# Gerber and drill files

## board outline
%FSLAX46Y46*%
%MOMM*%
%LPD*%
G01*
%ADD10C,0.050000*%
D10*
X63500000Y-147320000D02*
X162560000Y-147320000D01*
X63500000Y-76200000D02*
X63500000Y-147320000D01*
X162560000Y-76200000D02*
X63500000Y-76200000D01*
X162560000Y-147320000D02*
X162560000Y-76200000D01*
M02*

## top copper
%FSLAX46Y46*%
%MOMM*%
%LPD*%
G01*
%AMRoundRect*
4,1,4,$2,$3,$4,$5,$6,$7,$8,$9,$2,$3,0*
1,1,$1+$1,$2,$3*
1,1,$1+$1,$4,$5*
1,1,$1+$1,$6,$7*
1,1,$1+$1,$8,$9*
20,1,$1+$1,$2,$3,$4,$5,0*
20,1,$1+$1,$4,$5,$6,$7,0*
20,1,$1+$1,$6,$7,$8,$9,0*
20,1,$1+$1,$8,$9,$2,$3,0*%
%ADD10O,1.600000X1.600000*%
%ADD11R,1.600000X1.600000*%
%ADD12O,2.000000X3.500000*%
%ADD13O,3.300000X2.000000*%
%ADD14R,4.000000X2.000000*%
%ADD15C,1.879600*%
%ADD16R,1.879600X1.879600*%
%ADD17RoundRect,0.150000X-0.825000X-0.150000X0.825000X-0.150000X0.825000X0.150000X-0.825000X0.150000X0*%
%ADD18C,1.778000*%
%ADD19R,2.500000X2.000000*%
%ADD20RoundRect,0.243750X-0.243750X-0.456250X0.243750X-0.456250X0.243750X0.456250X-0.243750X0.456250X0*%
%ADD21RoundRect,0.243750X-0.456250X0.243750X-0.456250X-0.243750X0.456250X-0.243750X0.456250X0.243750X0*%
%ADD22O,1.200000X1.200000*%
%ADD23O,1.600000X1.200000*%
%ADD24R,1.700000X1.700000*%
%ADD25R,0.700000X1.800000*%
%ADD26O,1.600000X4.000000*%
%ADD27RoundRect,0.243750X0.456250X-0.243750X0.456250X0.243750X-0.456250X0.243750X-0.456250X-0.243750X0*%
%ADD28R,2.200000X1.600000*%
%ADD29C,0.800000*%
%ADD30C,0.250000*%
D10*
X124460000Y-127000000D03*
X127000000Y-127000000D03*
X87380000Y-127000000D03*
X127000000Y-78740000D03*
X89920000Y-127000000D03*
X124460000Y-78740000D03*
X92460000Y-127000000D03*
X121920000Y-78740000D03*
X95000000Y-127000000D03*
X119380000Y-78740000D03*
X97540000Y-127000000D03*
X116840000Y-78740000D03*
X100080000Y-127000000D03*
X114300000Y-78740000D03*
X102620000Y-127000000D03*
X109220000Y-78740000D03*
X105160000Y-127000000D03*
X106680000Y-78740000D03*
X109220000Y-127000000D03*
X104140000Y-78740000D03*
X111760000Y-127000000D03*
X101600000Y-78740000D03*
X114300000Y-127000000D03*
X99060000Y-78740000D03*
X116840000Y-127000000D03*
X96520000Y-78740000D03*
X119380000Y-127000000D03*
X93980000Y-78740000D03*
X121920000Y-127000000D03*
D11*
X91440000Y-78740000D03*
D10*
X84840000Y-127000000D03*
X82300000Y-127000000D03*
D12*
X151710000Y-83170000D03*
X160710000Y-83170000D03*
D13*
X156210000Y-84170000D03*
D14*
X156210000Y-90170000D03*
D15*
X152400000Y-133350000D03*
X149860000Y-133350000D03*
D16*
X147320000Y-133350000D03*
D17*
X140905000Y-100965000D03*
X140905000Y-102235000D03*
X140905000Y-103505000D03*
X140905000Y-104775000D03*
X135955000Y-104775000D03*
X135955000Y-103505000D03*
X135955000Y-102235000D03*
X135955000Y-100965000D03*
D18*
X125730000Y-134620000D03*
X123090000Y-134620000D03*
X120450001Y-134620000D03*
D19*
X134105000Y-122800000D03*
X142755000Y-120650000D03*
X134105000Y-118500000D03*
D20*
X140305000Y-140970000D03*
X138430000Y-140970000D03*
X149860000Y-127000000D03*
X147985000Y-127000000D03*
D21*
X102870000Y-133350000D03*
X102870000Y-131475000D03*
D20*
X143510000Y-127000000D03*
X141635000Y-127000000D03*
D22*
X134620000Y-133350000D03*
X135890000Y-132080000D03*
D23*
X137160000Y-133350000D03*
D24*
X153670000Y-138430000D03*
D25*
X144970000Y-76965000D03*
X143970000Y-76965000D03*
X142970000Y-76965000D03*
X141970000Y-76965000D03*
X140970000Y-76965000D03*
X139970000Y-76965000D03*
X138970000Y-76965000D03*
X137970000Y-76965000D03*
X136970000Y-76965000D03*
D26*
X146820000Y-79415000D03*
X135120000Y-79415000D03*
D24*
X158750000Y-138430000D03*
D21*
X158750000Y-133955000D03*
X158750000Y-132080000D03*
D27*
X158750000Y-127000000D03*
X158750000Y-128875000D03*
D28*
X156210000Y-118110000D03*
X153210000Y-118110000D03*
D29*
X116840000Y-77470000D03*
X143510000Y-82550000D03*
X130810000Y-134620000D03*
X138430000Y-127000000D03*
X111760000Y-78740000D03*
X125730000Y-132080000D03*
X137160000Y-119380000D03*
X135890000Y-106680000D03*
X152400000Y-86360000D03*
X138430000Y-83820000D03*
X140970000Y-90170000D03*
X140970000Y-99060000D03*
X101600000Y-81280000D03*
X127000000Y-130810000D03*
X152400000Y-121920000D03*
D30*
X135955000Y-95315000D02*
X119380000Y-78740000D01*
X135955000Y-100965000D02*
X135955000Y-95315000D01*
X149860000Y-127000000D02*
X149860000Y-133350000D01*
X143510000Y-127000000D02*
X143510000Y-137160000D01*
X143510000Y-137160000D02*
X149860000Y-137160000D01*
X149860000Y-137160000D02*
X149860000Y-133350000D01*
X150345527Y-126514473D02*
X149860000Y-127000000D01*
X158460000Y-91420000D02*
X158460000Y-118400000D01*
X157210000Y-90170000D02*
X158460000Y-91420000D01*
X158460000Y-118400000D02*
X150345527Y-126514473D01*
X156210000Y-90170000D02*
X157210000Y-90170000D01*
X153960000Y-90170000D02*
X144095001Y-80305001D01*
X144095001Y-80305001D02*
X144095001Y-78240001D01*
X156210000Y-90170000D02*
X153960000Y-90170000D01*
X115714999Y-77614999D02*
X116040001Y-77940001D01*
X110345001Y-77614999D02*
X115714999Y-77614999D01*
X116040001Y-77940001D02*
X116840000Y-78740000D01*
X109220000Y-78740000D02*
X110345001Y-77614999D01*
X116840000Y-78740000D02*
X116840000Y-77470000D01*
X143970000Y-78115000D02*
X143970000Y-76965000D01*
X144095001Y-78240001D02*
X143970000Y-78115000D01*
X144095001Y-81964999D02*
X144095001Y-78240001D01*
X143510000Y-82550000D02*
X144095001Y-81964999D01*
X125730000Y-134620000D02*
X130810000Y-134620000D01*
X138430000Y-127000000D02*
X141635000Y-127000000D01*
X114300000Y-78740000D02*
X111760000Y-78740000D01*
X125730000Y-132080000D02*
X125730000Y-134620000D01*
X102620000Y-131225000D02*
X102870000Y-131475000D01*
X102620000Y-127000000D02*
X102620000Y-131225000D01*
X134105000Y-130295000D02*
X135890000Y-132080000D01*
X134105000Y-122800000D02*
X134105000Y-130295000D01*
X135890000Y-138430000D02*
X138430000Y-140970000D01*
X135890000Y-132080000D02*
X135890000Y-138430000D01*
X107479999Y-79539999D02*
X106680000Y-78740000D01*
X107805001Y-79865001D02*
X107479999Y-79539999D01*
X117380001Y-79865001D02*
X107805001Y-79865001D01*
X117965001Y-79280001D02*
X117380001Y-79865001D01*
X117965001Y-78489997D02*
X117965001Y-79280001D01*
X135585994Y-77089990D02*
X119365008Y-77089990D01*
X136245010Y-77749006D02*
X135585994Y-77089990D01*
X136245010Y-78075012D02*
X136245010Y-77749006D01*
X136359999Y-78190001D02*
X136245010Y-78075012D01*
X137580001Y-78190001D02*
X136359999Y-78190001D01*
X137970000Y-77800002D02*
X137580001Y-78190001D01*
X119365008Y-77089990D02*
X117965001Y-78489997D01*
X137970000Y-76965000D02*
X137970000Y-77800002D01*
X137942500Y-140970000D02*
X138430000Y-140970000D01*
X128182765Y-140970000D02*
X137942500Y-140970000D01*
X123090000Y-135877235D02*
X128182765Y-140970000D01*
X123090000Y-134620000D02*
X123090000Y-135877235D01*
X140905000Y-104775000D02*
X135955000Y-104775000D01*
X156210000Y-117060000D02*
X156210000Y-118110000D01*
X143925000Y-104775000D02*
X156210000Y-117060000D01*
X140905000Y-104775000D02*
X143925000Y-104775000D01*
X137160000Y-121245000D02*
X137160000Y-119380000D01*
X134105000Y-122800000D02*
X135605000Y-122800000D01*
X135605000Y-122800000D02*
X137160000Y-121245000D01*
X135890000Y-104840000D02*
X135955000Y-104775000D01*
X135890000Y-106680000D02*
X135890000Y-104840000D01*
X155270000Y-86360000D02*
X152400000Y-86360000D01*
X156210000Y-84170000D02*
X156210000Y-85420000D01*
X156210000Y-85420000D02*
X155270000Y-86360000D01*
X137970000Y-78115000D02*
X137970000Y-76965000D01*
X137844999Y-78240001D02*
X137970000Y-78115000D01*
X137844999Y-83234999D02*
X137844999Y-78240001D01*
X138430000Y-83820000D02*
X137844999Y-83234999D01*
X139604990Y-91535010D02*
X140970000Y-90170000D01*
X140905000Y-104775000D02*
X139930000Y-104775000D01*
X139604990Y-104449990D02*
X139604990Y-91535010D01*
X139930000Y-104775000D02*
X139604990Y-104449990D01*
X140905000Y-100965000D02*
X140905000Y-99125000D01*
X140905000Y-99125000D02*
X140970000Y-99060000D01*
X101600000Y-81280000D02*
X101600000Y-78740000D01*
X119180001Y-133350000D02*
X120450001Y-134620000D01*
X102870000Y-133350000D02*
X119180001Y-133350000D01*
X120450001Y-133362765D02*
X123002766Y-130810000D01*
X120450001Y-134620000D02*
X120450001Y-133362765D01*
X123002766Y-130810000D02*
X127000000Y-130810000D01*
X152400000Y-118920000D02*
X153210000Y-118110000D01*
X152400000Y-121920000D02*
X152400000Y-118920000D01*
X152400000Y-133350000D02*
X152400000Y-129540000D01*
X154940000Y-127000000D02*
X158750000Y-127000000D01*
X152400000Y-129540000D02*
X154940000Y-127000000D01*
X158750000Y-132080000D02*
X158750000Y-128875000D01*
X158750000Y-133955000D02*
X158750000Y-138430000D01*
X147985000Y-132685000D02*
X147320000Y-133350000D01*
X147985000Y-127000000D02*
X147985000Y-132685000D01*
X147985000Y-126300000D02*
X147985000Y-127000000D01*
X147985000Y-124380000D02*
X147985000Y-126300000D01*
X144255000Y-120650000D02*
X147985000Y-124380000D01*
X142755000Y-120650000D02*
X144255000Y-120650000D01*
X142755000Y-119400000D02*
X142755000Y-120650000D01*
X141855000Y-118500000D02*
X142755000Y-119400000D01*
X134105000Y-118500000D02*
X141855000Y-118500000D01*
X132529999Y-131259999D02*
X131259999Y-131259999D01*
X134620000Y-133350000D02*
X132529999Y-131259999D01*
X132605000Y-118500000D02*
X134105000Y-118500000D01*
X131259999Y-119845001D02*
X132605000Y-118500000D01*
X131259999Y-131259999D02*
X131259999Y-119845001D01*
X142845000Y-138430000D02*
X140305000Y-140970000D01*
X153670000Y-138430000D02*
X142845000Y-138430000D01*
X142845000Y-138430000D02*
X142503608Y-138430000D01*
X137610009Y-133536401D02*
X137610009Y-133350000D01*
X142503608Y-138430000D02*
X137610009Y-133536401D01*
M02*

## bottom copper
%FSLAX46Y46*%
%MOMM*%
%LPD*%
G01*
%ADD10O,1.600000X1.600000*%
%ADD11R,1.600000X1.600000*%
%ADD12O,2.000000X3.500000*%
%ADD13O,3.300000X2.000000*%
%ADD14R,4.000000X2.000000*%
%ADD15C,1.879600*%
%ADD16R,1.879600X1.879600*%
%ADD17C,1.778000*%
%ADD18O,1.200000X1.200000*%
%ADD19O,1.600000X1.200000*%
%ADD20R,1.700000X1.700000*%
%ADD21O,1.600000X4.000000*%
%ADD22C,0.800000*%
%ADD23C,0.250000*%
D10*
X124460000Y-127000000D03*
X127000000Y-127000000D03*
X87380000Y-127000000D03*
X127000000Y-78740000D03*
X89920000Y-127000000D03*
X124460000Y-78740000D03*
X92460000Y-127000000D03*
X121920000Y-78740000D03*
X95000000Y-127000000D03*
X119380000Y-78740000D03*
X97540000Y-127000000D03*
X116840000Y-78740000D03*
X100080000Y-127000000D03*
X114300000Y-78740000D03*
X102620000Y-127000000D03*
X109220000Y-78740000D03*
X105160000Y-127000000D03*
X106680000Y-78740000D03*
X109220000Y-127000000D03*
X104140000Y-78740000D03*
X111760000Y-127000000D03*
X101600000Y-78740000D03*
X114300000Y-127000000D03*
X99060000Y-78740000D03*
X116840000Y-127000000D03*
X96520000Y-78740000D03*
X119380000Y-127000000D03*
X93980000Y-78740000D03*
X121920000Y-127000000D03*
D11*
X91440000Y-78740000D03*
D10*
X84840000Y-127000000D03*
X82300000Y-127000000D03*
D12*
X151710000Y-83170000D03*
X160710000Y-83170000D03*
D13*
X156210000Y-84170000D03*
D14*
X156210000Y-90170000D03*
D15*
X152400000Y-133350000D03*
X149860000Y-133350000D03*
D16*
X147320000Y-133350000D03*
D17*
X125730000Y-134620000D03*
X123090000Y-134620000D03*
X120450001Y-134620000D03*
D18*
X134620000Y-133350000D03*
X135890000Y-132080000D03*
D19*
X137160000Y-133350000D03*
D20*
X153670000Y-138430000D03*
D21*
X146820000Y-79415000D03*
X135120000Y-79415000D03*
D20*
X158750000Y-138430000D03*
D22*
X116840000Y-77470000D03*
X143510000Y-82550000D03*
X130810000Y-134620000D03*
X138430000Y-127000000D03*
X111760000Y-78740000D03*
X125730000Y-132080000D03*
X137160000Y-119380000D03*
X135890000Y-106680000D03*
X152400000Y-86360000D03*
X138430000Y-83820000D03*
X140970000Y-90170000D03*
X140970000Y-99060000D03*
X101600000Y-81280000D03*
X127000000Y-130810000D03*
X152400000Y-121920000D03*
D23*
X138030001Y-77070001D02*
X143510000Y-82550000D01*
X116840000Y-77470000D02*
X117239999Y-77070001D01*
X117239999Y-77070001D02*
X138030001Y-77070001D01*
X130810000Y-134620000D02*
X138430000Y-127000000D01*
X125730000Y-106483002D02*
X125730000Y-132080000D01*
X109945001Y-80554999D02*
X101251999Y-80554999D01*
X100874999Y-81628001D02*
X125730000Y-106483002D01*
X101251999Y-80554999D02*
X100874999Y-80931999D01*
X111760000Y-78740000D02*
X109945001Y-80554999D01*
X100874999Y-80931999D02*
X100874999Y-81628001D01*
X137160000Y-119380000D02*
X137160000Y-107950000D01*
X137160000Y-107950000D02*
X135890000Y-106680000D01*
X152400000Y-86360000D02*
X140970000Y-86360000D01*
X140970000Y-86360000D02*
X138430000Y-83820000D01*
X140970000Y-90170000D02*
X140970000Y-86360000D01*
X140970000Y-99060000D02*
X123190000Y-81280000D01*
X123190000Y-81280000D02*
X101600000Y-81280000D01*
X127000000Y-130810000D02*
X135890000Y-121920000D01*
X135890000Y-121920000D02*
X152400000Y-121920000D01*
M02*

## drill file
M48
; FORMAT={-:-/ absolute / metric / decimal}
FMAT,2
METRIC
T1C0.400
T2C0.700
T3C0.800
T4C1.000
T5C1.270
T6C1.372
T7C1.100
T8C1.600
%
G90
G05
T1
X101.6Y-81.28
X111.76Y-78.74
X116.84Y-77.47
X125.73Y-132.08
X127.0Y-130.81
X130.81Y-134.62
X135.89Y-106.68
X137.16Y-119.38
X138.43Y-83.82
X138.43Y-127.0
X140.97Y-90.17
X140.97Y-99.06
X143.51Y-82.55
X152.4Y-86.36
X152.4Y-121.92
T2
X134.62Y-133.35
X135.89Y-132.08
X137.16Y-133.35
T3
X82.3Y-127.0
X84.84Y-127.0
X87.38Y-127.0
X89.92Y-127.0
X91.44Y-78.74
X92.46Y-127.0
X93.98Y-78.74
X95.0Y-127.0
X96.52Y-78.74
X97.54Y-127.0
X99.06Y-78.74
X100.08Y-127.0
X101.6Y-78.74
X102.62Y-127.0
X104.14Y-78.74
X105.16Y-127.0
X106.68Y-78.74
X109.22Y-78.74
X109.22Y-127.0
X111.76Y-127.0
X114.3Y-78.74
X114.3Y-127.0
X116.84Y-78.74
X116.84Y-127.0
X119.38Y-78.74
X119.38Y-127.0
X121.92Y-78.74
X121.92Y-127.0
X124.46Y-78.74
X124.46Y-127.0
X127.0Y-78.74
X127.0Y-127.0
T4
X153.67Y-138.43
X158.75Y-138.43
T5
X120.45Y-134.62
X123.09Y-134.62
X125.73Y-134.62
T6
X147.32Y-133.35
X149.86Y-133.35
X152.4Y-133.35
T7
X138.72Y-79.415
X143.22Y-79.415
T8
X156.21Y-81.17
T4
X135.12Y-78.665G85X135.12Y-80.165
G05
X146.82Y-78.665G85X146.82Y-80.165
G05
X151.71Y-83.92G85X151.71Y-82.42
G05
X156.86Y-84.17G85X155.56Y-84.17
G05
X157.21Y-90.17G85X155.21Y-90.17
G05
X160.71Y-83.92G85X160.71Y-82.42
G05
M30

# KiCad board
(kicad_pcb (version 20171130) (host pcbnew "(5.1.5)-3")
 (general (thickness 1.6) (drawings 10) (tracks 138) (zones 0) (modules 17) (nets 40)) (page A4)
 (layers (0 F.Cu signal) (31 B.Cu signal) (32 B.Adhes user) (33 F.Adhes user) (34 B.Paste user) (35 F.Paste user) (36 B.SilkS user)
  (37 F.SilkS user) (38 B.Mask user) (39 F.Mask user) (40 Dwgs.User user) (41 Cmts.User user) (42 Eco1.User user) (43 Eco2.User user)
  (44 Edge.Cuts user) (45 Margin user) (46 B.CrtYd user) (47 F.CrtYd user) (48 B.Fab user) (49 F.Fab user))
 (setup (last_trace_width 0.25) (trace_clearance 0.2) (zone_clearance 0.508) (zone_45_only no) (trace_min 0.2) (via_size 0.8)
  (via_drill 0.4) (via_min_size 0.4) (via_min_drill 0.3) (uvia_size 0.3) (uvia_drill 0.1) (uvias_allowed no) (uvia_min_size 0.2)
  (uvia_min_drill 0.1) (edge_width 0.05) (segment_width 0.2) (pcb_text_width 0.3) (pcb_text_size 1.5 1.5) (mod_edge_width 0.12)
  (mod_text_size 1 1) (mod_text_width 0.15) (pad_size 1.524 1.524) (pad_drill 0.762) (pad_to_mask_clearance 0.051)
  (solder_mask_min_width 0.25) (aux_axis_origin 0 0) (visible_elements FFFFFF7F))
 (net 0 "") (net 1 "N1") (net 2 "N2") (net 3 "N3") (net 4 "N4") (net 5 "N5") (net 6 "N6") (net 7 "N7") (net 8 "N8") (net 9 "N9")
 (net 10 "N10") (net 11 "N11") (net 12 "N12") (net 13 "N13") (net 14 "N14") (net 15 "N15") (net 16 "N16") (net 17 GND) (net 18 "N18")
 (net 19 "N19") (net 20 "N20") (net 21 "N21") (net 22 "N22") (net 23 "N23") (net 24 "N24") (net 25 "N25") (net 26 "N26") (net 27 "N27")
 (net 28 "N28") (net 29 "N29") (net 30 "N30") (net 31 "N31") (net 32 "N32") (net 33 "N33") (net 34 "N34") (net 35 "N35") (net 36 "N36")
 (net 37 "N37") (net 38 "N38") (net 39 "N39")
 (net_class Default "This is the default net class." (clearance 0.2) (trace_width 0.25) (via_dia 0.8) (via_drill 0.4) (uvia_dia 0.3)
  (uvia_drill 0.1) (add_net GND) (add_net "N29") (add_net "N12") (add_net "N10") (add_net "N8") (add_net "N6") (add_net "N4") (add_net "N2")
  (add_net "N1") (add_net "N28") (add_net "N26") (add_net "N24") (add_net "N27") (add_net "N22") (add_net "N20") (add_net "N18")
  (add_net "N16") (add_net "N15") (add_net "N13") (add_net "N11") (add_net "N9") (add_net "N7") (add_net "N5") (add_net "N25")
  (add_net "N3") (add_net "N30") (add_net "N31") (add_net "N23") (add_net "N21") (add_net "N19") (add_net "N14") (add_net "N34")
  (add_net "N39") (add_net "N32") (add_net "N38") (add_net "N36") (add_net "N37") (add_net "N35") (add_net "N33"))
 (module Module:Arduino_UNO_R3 (layer F.Cu) (at 91.44 78.74)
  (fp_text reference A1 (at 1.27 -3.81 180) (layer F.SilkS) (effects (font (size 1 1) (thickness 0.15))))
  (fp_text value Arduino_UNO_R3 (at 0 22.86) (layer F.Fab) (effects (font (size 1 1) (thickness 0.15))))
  (pad 16 thru_hole oval (at 33.02 48.26 90) (size 1.6 1.6) (drill 0.8) (layers *.Cu *.Mask) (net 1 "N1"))
  (pad 15 thru_hole oval (at 35.56 48.26 90) (size 1.6 1.6) (drill 0.8) (layers *.Cu *.Mask) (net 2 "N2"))
  (pad 30 thru_hole oval (at -4.06 48.26 90) (size 1.6 1.6) (drill 0.8) (layers *.Cu *.Mask) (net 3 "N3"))
  (pad 14 thru_hole oval (at 35.56 0 90) (size 1.6 1.6) (drill 0.8) (layers *.Cu *.Mask) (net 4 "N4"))
  (pad 29 thru_hole oval (at -1.52 48.26 90) (size 1.6 1.6) (drill 0.8) (layers *.Cu *.Mask) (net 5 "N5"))
  (pad 13 thru_hole oval (at 33.02 0 90) (size 1.6 1.6) (drill 0.8) (layers *.Cu *.Mask) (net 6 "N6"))
  (pad 28 thru_hole oval (at 1.02 48.26 90) (size 1.6 1.6) (drill 0.8) (layers *.Cu *.Mask) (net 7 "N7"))
  (pad 12 thru_hole oval (at 30.48 0 90) (size 1.6 1.6) (drill 0.8) (layers *.Cu *.Mask) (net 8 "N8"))
  (pad 27 thru_hole oval (at 3.56 48.26 90) (size 1.6 1.6) (drill 0.8) (layers *.Cu *.Mask) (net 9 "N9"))
  (pad 11 thru_hole oval (at 27.94 0 90) (size 1.6 1.6) (drill 0.8) (layers *.Cu *.Mask) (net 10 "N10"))
  (pad 26 thru_hole oval (at 6.1 48.26 90) (size 1.6 1.6) (drill 0.8) (layers *.Cu *.Mask) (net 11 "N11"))
  (pad 10 thru_hole oval (at 25.4 0 90) (size 1.6 1.6) (drill 0.8) (layers *.Cu *.Mask) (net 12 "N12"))
  (pad 25 thru_hole oval (at 8.64 48.26 90) (size 1.6 1.6) (drill 0.8) (layers *.Cu *.Mask) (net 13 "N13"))
  (pad 9 thru_hole oval (at 22.86 0 90) (size 1.6 1.6) (drill 0.8) (layers *.Cu *.Mask) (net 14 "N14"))
  (pad 24 thru_hole oval (at 11.18 48.26 90) (size 1.6 1.6) (drill 0.8) (layers *.Cu *.Mask) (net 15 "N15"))
  (pad 8 thru_hole oval (at 17.78 0 90) (size 1.6 1.6) (drill 0.8) (layers *.Cu *.Mask) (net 12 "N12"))
  (pad 23 thru_hole oval (at 13.72 48.26 90) (size 1.6 1.6) (drill 0.8) (layers *.Cu *.Mask) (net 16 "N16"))
  (pad 7 thru_hole oval (at 15.24 0 90) (size 1.6 1.6) (drill 0.8) (layers *.Cu *.Mask) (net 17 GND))
  (pad 22 thru_hole oval (at 17.78 48.26 90) (size 1.6 1.6) (drill 0.8) (layers *.Cu *.Mask) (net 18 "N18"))
  (pad 6 thru_hole oval (at 12.7 0 90) (size 1.6 1.6) (drill 0.8) (layers *.Cu *.Mask) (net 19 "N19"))
  (pad 21 thru_hole oval (at 20.32 48.26 90) (size 1.6 1.6) (drill 0.8) (layers *.Cu *.Mask) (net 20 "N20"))
  (pad 5 thru_hole oval (at 10.16 0 90) (size 1.6 1.6) (drill 0.8) (layers *.Cu *.Mask) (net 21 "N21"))
  (pad 20 thru_hole oval (at 22.86 48.26 90) (size 1.6 1.6) (drill 0.8) (layers *.Cu *.Mask) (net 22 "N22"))
  (pad 4 thru_hole oval (at 7.62 0 90) (size 1.6 1.6) (drill 0.8) (layers *.Cu *.Mask) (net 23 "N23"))
  (pad 19 thru_hole oval (at 25.4 48.26 90) (size 1.6 1.6) (drill 0.8) (layers *.Cu *.Mask) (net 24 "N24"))
  (pad 3 thru_hole oval (at 5.08 0 90) (size 1.6 1.6) (drill 0.8) (layers *.Cu *.Mask) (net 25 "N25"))
  (pad 18 thru_hole oval (at 27.94 48.26 90) (size 1.6 1.6) (drill 0.8) (layers *.Cu *.Mask) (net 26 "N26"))
  (pad 2 thru_hole oval (at 2.54 0 90) (size 1.6 1.6) (drill 0.8) (layers *.Cu *.Mask) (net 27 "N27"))
  (pad 17 thru_hole oval (at 30.48 48.26 90) (size 1.6 1.6) (drill 0.8) (layers *.Cu *.Mask) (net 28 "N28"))
  (pad 1 thru_hole rect (at 0 0 90) (size 1.6 1.6) (drill 0.8) (layers *.Cu *.Mask) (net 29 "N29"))
  (pad 31 thru_hole oval (at -6.6 48.26 90) (size 1.6 1.6) (drill 0.8) (layers *.Cu *.Mask) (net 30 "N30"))
  (pad 32 thru_hole oval (at -9.14 48.26 90) (size 1.6 1.6) (drill 0.8) (layers *.Cu *.Mask) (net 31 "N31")))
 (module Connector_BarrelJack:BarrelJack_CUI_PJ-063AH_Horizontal (layer F.Cu) (at 156.21 90.17 180)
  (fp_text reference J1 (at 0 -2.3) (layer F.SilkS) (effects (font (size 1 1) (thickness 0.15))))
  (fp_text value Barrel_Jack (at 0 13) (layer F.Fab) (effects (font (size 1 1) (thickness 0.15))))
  (pad "" np_thru_hole circle (at 0 9 180) (size 1.6 1.6) (drill 1.6) (layers *.Cu *.Mask))
  (pad MP thru_hole oval (at 4.5 7 180) (size 2 3.5) (drill oval 1 2.5) (layers *.Cu *.Mask))
  (pad MP thru_hole oval (at -4.5 7 180) (size 2 3.5) (drill oval 1 2.5) (layers *.Cu *.Mask))
  (pad 2 thru_hole oval (at 0 6 180) (size 3.3 2) (drill oval 2.3 1) (layers *.Cu *.Mask) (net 17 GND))
  (pad 1 thru_hole rect (at 0 0 180) (size 4 2) (drill oval 3 1) (layers *.Cu *.Mask) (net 12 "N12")))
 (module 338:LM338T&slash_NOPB (layer F.Cu) (at 147.32 133.35)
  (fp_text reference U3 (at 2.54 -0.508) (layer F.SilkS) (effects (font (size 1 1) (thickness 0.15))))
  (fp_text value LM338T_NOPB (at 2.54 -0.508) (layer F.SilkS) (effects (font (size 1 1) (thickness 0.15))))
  (pad 3 thru_hole circle (at 5.08 0) (size 1.8796 1.8796) (drill 1.3716) (layers *.Cu *.Mask) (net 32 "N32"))
  (pad 2 thru_hole circle (at 2.54 0) (size 1.8796 1.8796) (drill 1.3716) (layers *.Cu *.Mask) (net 12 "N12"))
  (pad 1 thru_hole rect (at 0 0) (size 1.8796 1.8796) (drill 1.3716) (layers *.Cu *.Mask) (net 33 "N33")))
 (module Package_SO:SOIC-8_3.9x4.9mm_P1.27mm (layer F.Cu) (at 138.43 102.87)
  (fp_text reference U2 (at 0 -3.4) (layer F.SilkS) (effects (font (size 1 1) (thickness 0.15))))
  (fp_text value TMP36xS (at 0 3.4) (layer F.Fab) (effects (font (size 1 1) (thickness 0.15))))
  (pad 8 smd roundrect (at 2.475 -1.905) (size 1.95 0.6) (layers F.Cu F.Paste F.Mask) (roundrect_rratio 0.25) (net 21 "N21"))
  (pad 7 smd roundrect (at 2.475 -0.635) (size 1.95 0.6) (layers F.Cu F.Paste F.Mask) (roundrect_rratio 0.25))
  (pad 6 smd roundrect (at 2.475 0.635) (size 1.95 0.6) (layers F.Cu F.Paste F.Mask) (roundrect_rratio 0.25))
  (pad 5 smd roundrect (at 2.475 1.905) (size 1.95 0.6) (layers F.Cu F.Paste F.Mask) (roundrect_rratio 0.25) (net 17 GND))
  (pad 4 smd roundrect (at -2.475 1.905) (size 1.95 0.6) (layers F.Cu F.Paste F.Mask) (roundrect_rratio 0.25) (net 17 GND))
  (pad 3 smd roundrect (at -2.475 0.635) (size 1.95 0.6) (layers F.Cu F.Paste F.Mask) (roundrect_rratio 0.25))
  (pad 2 smd roundrect (at -2.475 -0.635) (size 1.95 0.6) (layers F.Cu F.Paste F.Mask) (roundrect_rratio 0.25))
  (pad 1 smd roundrect (at -2.475 -1.905) (size 1.95 0.6) (layers F.Cu F.Paste F.Mask) (roundrect_rratio 0.25) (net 10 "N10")))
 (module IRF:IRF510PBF (layer F.Cu) (at 125.73 134.62)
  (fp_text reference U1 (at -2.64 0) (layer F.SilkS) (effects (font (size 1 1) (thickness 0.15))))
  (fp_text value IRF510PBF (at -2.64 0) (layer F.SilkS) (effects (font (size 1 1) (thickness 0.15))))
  (pad 3 thru_hole circle (at 0 0) (size 1.778 1.778) (drill 1.27) (layers *.Cu *.Mask) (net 14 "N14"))
  (pad 2 thru_hole circle (at -2.64 0) (size 1.778 1.778) (drill 1.27) (layers *.Cu *.Mask) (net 17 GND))
  (pad 1 thru_hole circle (at -5.279999 0) (size 1.778 1.778) (drill 1.27) (layers *.Cu *.Mask) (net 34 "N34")))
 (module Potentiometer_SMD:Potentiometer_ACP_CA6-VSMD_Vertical (layer F.Cu) (at 138.43 120.65)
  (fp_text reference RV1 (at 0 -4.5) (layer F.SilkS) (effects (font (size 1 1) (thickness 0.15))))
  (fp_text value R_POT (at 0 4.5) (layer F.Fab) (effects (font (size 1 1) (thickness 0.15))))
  (pad 1 smd rect (at -4.325 2.15) (size 2.5 2) (layers F.Cu F.Paste F.Mask) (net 17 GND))
  (pad 2 smd rect (at 4.325 0) (size 2.5 2) (layers F.Cu F.Paste F.Mask) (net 33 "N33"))
  (pad 3 smd rect (at -4.325 -2.15) (size 2.5 2) (layers F.Cu F.Paste F.Mask) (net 33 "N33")))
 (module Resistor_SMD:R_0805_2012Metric (layer F.Cu) (at 139.3675 140.97)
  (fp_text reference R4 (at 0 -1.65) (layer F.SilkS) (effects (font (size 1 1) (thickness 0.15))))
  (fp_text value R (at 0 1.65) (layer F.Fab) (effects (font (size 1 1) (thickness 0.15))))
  (pad 2 smd roundrect (at 0.9375 0) (size 0.975 1.4) (layers F.Cu F.Paste F.Mask) (roundrect_rratio 0.25) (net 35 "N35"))
  (pad 1 smd roundrect (at -0.9375 0) (size 0.975 1.4) (layers F.Cu F.Paste F.Mask) (roundrect_rratio 0.25) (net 17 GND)))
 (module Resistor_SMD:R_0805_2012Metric (layer F.Cu) (at 148.9225 127)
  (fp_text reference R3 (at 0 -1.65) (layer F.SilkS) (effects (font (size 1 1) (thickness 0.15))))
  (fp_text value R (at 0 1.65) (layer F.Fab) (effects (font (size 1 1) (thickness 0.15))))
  (pad 2 smd roundrect (at 0.9375 0) (size 0.975 1.4) (layers F.Cu F.Paste F.Mask) (roundrect_rratio 0.25) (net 12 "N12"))
  (pad 1 smd roundrect (at -0.9375 0) (size 0.975 1.4) (layers F.Cu F.Paste F.Mask) (roundrect_rratio 0.25) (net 33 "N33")))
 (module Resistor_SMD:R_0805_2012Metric (layer F.Cu) (at 102.87 132.4125 270)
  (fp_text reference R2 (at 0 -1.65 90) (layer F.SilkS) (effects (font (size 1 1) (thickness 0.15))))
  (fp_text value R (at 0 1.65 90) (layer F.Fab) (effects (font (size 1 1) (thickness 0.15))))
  (pad 2 smd roundrect (at 0.9375 0 270) (size 0.975 1.4) (layers F.Cu F.Paste F.Mask) (roundrect_rratio 0.25) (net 34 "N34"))
  (pad 1 smd roundrect (at -0.9375 0 270) (size 0.975 1.4) (layers F.Cu F.Paste F.Mask) (roundrect_rratio 0.25) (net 15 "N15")))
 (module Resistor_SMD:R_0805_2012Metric (layer F.Cu) (at 142.5725 127)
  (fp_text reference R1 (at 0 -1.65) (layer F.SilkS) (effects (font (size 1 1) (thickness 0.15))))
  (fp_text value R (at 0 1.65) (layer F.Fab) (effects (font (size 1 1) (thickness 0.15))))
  (pad 2 smd roundrect (at 0.9375 0) (size 0.975 1.4) (layers F.Cu F.Paste F.Mask) (roundrect_rratio 0.25) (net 12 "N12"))
  (pad 1 smd roundrect (at -0.9375 0) (size 0.975 1.4) (layers F.Cu F.Paste F.Mask) (roundrect_rratio 0.25) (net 14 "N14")))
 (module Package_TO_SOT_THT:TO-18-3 (layer F.Cu) (at 137.16 133.35 180)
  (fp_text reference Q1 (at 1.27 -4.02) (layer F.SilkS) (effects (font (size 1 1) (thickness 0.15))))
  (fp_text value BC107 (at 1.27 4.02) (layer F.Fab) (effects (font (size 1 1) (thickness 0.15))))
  (pad 3 thru_hole oval (at 2.54 0 180) (size 1.2 1.2) (drill 0.7) (layers *.Cu *.Mask) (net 33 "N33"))
  (pad 2 thru_hole oval (at 1.27 1.27 180) (size 1.2 1.2) (drill 0.7) (layers *.Cu *.Mask) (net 17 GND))
  (pad 1 thru_hole oval (at 0 0 180) (size 1.6 1.2) (drill 0.7) (layers *.Cu *.Mask) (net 35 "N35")))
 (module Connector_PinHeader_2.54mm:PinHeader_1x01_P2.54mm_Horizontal (layer F.Cu) (at 153.67 138.43 270)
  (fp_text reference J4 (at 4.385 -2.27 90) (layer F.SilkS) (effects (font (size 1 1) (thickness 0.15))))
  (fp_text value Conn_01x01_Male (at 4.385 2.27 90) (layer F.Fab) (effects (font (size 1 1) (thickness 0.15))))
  (pad 1 thru_hole rect (at 0 0 270) (size 1.7 1.7) (drill 1) (layers *.Cu *.Mask) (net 35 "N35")))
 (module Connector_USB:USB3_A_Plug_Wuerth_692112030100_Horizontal (layer F.Cu) (at 140.97 78.74 270)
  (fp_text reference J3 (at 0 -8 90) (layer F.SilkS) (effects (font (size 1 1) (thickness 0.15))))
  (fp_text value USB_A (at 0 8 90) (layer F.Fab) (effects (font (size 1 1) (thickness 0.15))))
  (pad "" np_thru_hole circle (at 0.675 -2.25) (size 1.1 1.1) (drill 1.1) (layers *.Cu *.Mask))
  (pad "" np_thru_hole circle (at 0.675 2.25) (size 1.1 1.1) (drill 1.1) (layers *.Cu *.Mask))
  (pad 9 smd rect (at -1.775 -4 270) (size 1.8 0.7) (layers F.Cu F.Paste F.Mask))
  (pad 1 smd rect (at -1.775 -3) (size 0.7 1.8) (layers F.Cu F.Paste F.Mask) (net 12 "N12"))
  (pad 8 smd rect (at -1.775 -2) (size 0.7 1.8) (layers F.Cu F.Paste F.Mask))
  (pad 2 smd rect (at -1.775 -1) (size 0.7 1.8) (layers F.Cu F.Paste F.Mask) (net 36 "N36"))
  (pad 7 smd rect (at -1.775 0) (size 0.7 1.8) (layers F.Cu F.Paste F.Mask))
  (pad 3 smd rect (at -1.775 1) (size 0.7 1.8) (layers F.Cu F.Paste F.Mask) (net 36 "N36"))
  (pad 6 smd rect (at -1.775 2) (size 0.7 1.8) (layers F.Cu F.Paste F.Mask))
  (pad 4 smd rect (at -1.775 3) (size 0.7 1.8) (layers F.Cu F.Paste F.Mask) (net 17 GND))
  (pad 5 smd rect (at -1.775 4) (size 0.7 1.8) (layers F.Cu F.Paste F.Mask) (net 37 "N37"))
  (pad 10 thru_hole oval (at 0.675 -5.85) (size 1.6 4) (drill oval 1 2.5) (layers *.Cu *.Mask))
  (pad 10 thru_hole oval (at 0.675 5.85) (size 1.6 4) (drill oval 1 2.5) (layers *.Cu *.Mask)))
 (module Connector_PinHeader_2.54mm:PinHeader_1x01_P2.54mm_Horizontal (layer F.Cu) (at 158.75 138.43 270)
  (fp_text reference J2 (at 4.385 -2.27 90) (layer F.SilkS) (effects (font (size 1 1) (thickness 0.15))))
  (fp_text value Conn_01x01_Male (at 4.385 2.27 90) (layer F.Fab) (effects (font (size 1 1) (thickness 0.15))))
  (pad 1 thru_hole rect (at 0 0 270) (size 1.7 1.7) (drill 1) (layers *.Cu *.Mask) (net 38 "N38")))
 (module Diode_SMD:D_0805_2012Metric (layer F.Cu) (at 158.75 133.0175 270)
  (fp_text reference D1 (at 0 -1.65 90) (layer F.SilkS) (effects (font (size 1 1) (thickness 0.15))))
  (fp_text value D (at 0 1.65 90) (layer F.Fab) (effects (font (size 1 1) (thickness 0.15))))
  (pad 2 smd roundrect (at 0.9375 0 270) (size 0.975 1.4) (layers F.Cu F.Paste F.Mask) (roundrect_rratio 0.25) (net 38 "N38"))
  (pad 1 smd roundrect (at -0.9375 0 270) (size 0.975 1.4) (layers F.Cu F.Paste F.Mask) (roundrect_rratio 0.25) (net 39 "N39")))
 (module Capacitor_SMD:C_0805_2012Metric (layer F.Cu) (at 158.75 127.9375 90)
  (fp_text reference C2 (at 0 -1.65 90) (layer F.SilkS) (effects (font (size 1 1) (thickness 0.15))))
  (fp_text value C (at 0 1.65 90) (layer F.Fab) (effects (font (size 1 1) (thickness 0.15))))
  (pad 2 smd roundrect (at 0.9375 0 90) (size 0.975 1.4) (layers F.Cu F.Paste F.Mask) (roundrect_rratio 0.25) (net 32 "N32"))
  (pad 1 smd roundrect (at -0.9375 0 90) (size 0.975 1.4) (layers F.Cu F.Paste F.Mask) (roundrect_rratio 0.25) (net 39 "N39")))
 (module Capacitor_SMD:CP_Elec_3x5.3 (layer F.Cu) (at 154.71 118.11)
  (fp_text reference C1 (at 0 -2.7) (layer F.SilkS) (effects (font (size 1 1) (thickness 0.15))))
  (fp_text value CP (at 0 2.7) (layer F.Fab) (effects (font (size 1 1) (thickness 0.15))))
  (pad 2 smd rect (at 1.5 0) (size 2.2 1.6) (layers F.Cu F.Paste F.Mask) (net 17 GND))
  (pad 1 smd rect (at -1.5 0) (size 2.2 1.6) (layers F.Cu F.Paste F.Mask) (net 34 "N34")))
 (gr_line (start 63.5 147.32) (end 162.56 147.32) (layer Edge.Cuts) (width 0.05))
 (gr_line (start 63.5 76.2) (end 63.5 147.32) (layer Edge.Cuts) (width 0.05))
 (gr_line (start 162.56 76.2) (end 63.5 76.2) (layer Edge.Cuts) (width 0.05))
 (gr_line (start 162.56 147.32) (end 162.56 76.2) (layer Edge.Cuts) (width 0.05))
 (segment (start 135.955 95.315) (end 119.38 78.74) (width 0.25) (layer F.Cu) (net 10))
 (segment (start 135.955 100.965) (end 135.955 95.315) (width 0.25) (layer F.Cu) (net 10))
 (segment (start 149.86 127) (end 149.86 133.35) (width 0.25) (layer F.Cu) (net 12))
 (segment (start 143.51 127) (end 143.51 137.16) (width 0.25) (layer F.Cu) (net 12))
 (segment (start 143.51 137.16) (end 149.86 137.16) (width 0.25) (layer F.Cu) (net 12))
 (segment (start 149.86 137.16) (end 149.86 133.35) (width 0.25) (layer F.Cu) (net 12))
 (segment (start 150.345527 126.514473) (end 149.86 127) (width 0.25) (layer F.Cu) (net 12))
 (segment (start 158.46 91.42) (end 158.46 118.4) (width 0.25) (layer F.Cu) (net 12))
 (segment (start 157.21 90.17) (end 158.46 91.42) (width 0.25) (layer F.Cu) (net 12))
 (segment (start 158.46 118.4) (end 150.345527 126.514473) (width 0.25) (layer F.Cu) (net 12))
 (segment (start 156.21 90.17) (end 157.21 90.17) (width 0.25) (layer F.Cu) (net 12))
 (segment (start 153.96 90.17) (end 144.095001 80.305001) (width 0.25) (layer F.Cu) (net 12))
 (segment (start 144.095001 80.305001) (end 144.095001 78.240001) (width 0.25) (layer F.Cu) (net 12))
 (segment (start 156.21 90.17) (end 153.96 90.17) (width 0.25) (layer F.Cu) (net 12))
 (segment (start 115.714999 77.614999) (end 116.040001 77.940001) (width 0.25) (layer F.Cu) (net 12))
 (segment (start 110.345001 77.614999) (end 115.714999 77.614999) (width 0.25) (layer F.Cu) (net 12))
 (segment (start 116.040001 77.940001) (end 116.84 78.74) (width 0.25) (layer F.Cu) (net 12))
 (segment (start 109.22 78.74) (end 110.345001 77.614999) (width 0.25) (layer F.Cu) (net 12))
 (via (at 116.84 77.47) (size 0.8) (drill 0.4) (layers F.Cu B.Cu) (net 12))
 (segment (start 116.84 78.74) (end 116.84 77.47) (width 0.25) (layer F.Cu) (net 12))
 (via (at 143.51 82.55) (size 0.8) (drill 0.4) (layers F.Cu B.Cu) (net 12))
 (segment (start 138.030001 77.070001) (end 143.51 82.55) (width 0.25) (layer B.Cu) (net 12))
 (segment (start 116.84 77.47) (end 117.239999 77.070001) (width 0.25) (layer B.Cu) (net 12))
 (segment (start 117.239999 77.070001) (end 138.030001 77.070001) (width 0.25) (layer B.Cu) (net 12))
 (segment (start 143.97 78.115) (end 143.97 76.965) (width 0.25) (layer F.Cu) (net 12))
 (segment (start 144.095001 78.240001) (end 143.97 78.115) (width 0.25) (layer F.Cu) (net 12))
 (segment (start 144.095001 81.964999) (end 144.095001 78.240001) (width 0.25) (layer F.Cu) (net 12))
 (segment (start 143.51 82.55) (end 144.095001 81.964999) (width 0.25) (layer F.Cu) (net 12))
 (via (at 130.81 134.62) (size 0.8) (drill 0.4) (layers F.Cu B.Cu) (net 14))
 (segment (start 125.73 134.62) (end 130.81 134.62) (width 0.25) (layer F.Cu) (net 14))
 (via (at 138.43 127) (size 0.8) (drill 0.4) (layers F.Cu B.Cu) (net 14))
 (segment (start 130.81 134.62) (end 138.43 127) (width 0.25) (layer B.Cu) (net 14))
 (segment (start 138.43 127) (end 141.635 127) (width 0.25) (layer F.Cu) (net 14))
 (via (at 111.76 78.74) (size 0.8) (drill 0.4) (layers F.Cu B.Cu) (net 14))
 (segment (start 114.3 78.74) (end 111.76 78.74) (width 0.25) (layer F.Cu) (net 14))
 (via (at 125.73 132.08) (size 0.8) (drill 0.4) (layers F.Cu B.Cu) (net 14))
 (segment (start 125.73 106.483002) (end 125.73 132.08) (width 0.25) (layer B.Cu) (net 14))
 (segment (start 109.945001 80.554999) (end 101.251999 80.554999) (width 0.25) (layer B.Cu) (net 14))
 (segment (start 100.874999 81.628001) (end 125.73 106.483002) (width 0.25) (layer B.Cu) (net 14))
 (segment (start 101.251999 80.554999) (end 100.874999 80.931999) (width 0.25) (layer B.Cu) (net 14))
 (segment (start 111.76 78.74) (end 109.945001 80.554999) (width 0.25) (layer B.Cu) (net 14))
 (segment (start 100.874999 80.931999) (end 100.874999 81.628001) (width 0.25) (layer B.Cu) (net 14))
 (segment (start 125.73 132.08) (end 125.73 134.62) (width 0.25) (layer F.Cu) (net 14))
 (segment (start 102.62 131.225) (end 102.87 131.475) (width 0.25) (layer F.Cu) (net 15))
 (segment (start 102.62 127) (end 102.62 131.225) (width 0.25) (layer F.Cu) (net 15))
 (segment (start 134.105 130.295) (end 135.89 132.08) (width 0.25) (layer F.Cu) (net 17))
 (segment (start 134.105 122.8) (end 134.105 130.295) (width 0.25) (layer F.Cu) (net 17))
 (segment (start 135.89 138.43) (end 138.43 140.97) (width 0.25) (layer F.Cu) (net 17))
 (segment (start 135.89 132.08) (end 135.89 138.43) (width 0.25) (layer F.Cu) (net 17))
 (segment (start 107.479999 79.539999) (end 106.68 78.74) (width 0.25) (layer F.Cu) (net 17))
 (segment (start 107.805001 79.865001) (end 107.479999 79.539999) (width 0.25) (layer F.Cu) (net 17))
 (segment (start 117.380001 79.865001) (end 107.805001 79.865001) (width 0.25) (layer F.Cu) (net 17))
 (segment (start 117.965001 79.280001) (end 117.380001 79.865001) (width 0.25) (layer F.Cu) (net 17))
 (segment (start 117.965001 78.489997) (end 117.965001 79.280001) (width 0.25) (layer F.Cu) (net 17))
 (segment (start 135.585994 77.08999) (end 119.365008 77.08999) (width 0.25) (layer F.Cu) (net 17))
 (segment (start 136.24501 77.749006) (end 135.585994 77.08999) (width 0.25) (layer F.Cu) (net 17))
 (segment (start 136.24501 78.075012) (end 136.24501 77.749006) (width 0.25) (layer F.Cu) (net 17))
 (segment (start 136.359999 78.190001) (end 136.24501 78.075012) (width 0.25) (layer F.Cu) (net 17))
 (segment (start 137.580001 78.190001) (end 136.359999 78.190001) (width 0.25) (layer F.Cu) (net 17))
 (segment (start 137.97 77.800002) (end 137.580001 78.190001) (width 0.25) (layer F.Cu) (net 17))
 (segment (start 119.365008 77.08999) (end 117.965001 78.489997) (width 0.25) (layer F.Cu) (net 17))
 (segment (start 137.97 76.965) (end 137.97 77.800002) (width 0.25) (layer F.Cu) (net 17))
 (segment (start 137.9425 140.97) (end 138.43 140.97) (width 0.25) (layer F.Cu) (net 17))
 (segment (start 128.182765 140.97) (end 137.9425 140.97) (width 0.25) (layer F.Cu) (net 17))
 (segment (start 123.09 135.877235) (end 128.182765 140.97) (width 0.25) (layer F.Cu) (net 17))
 (segment (start 123.09 134.62) (end 123.09 135.877235) (width 0.25) (layer F.Cu) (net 17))
 (segment (start 140.905 104.775) (end 135.955 104.775) (width 0.25) (layer F.Cu) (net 17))
 (segment (start 156.21 117.06) (end 156.21 118.11) (width 0.25) (layer F.Cu) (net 17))
 (segment (start 143.925 104.775) (end 156.21 117.06) (width 0.25) (layer F.Cu) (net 17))
 (segment (start 140.905 104.775) (end 143.925 104.775) (width 0.25) (layer F.Cu) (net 17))
 (via (at 137.16 119.38) (size 0.8) (drill 0.4) (layers F.Cu B.Cu) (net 17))
 (segment (start 137.16 121.245) (end 137.16 119.38) (width 0.25) (layer F.Cu) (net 17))
 (segment (start 134.105 122.8) (end 135.605 122.8) (width 0.25) (layer F.Cu) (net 17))
 (segment (start 135.605 122.8) (end 137.16 121.245) (width 0.25) (layer F.Cu) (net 17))
 (segment (start 137.16 119.38) (end 137.16 107.95) (width 0.25) (layer B.Cu) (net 17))
 (via (at 135.89 106.68) (size 0.8) (drill 0.4) (layers F.Cu B.Cu) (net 17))
 (segment (start 137.16 107.95) (end 135.89 106.68) (width 0.25) (layer B.Cu) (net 17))
 (segment (start 135.89 104.84) (end 135.955 104.775) (width 0.25) (layer F.Cu) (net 17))
 (segment (start 135.89 106.68) (end 135.89 104.84) (width 0.25) (layer F.Cu) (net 17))
 (via (at 152.4 86.36) (size 0.8) (drill 0.4) (layers F.Cu B.Cu) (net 17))
 (segment (start 155.27 86.36) (end 152.4 86.36) (width 0.25) (layer F.Cu) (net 17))
 (segment (start 156.21 84.17) (end 156.21 85.42) (width 0.25) (layer F.Cu) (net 17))
 (segment (start 156.21 85.42) (end 155.27 86.36) (width 0.25) (layer F.Cu) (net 17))
 (via (at 138.43 83.82) (size 0.8) (drill 0.4) (layers F.Cu B.Cu) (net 17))
 (segment (start 152.4 86.36) (end 140.97 86.36) (width 0.25) (layer B.Cu) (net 17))
 (segment (start 140.97 86.36) (end 138.43 83.82) (width 0.25) (layer B.Cu) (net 17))
 (segment (start 137.97 78.115) (end 137.97 76.965) (width 0.25) (layer F.Cu) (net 17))
 (segment (start 137.844999 78.240001) (end 137.97 78.115) (width 0.25) (layer F.Cu) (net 17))
 (segment (start 137.844999 83.234999) (end 137.844999 78.240001) (width 0.25) (layer F.Cu) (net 17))
 (segment (start 138.43 83.82) (end 137.844999 83.234999) (width 0.25) (layer F.Cu) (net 17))
 (via (at 140.97 90.17) (size 0.8) (drill 0.4) (layers F.Cu B.Cu) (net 17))
 (segment (start 139.60499 91.53501) (end 140.97 90.17) (width 0.25) (layer F.Cu) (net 17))
 (segment (start 140.905 104.775) (end 139.93 104.775) (width 0.25) (layer F.Cu) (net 17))
 (segment (start 139.60499 104.44999) (end 139.60499 91.53501) (width 0.25) (layer F.Cu) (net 17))
 (segment (start 139.93 104.775) (end 139.60499 104.44999) (width 0.25) (layer F.Cu) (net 17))
 (segment (start 140.97 90.17) (end 140.97 86.36) (width 0.25) (layer B.Cu) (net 17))
 (via (at 140.97 99.06) (size 0.8) (drill 0.4) (layers F.Cu B.Cu) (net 21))
 (segment (start 140.905 100.965) (end 140.905 99.125) (width 0.25) (layer F.Cu) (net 21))
 (segment (start 140.905 99.125) (end 140.97 99.06) (width 0.25) (layer F.Cu) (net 21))
 (via (at 101.6 81.28) (size 0.8) (drill 0.4) (layers F.Cu B.Cu) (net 21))
 (segment (start 140.97 99.06) (end 123.19 81.28) (width 0.25) (layer B.Cu) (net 21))
 (segment (start 123.19 81.28) (end 101.6 81.28) (width 0.25) (layer B.Cu) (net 21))
 (segment (start 101.6 81.28) (end 101.6 78.74) (width 0.25) (layer F.Cu) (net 21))
 (segment (start 119.180001 133.35) (end 120.450001 134.62) (width 0.25) (layer F.Cu) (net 34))
 (segment (start 102.87 133.35) (end 119.180001 133.35) (width 0.25) (layer F.Cu) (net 34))
 (segment (start 120.450001 133.362765) (end 123.002766 130.81) (width 0.25) (layer F.Cu) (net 34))
 (segment (start 120.450001 134.62) (end 120.450001 133.362765) (width 0.25) (layer F.Cu) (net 34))
 (via (at 127 130.81) (size 0.8) (drill 0.4) (layers F.Cu B.Cu) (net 34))
 (segment (start 123.002766 130.81) (end 127 130.81) (width 0.25) (layer F.Cu) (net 34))
 (via (at 152.4 121.92) (size 0.8) (drill 0.4) (layers F.Cu B.Cu) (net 34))
 (segment (start 127 130.81) (end 135.89 121.92) (width 0.25) (layer B.Cu) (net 34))
 (segment (start 135.89 121.92) (end 152.4 121.92) (width 0.25) (layer B.Cu) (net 34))
 (segment (start 152.4 118.92) (end 153.21 118.11) (width 0.25) (layer F.Cu) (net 34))
 (segment (start 152.4 121.92) (end 152.4 118.92) (width 0.25) (layer F.Cu) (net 34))
 (segment (start 152.4 133.35) (end 152.4 129.54) (width 0.25) (layer F.Cu) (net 32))
 (segment (start 154.94 127) (end 158.75 127) (width 0.25) (layer F.Cu) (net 32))
 (segment (start 152.4 129.54) (end 154.94 127) (width 0.25) (layer F.Cu) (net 32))
 (segment (start 158.75 132.08) (end 158.75 128.875) (width 0.25) (layer F.Cu) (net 39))
 (segment (start 158.75 133.955) (end 158.75 138.43) (width 0.25) (layer F.Cu) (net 38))
 (segment (start 147.985 132.685) (end 147.32 133.35) (width 0.25) (layer F.Cu) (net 33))
 (segment (start 147.985 127) (end 147.985 132.685) (width 0.25) (layer F.Cu) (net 33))
 (segment (start 147.985 126.3) (end 147.985 127) (width 0.25) (layer F.Cu) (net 33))
 (segment (start 147.985 124.38) (end 147.985 126.3) (width 0.25) (layer F.Cu) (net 33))
 (segment (start 144.255 120.65) (end 147.985 124.38) (width 0.25) (layer F.Cu) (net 33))
 (segment (start 142.755 120.65) (end 144.255 120.65) (width 0.25) (layer F.Cu) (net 33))
 (segment (start 142.755 119.4) (end 142.755 120.65) (width 0.25) (layer F.Cu) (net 33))
 (segment (start 141.855 118.5) (end 142.755 119.4) (width 0.25) (layer F.Cu) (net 33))
 (segment (start 134.105 118.5) (end 141.855 118.5) (width 0.25) (layer F.Cu) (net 33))
 (segment (start 132.529999 131.259999) (end 131.259999 131.259999) (width 0.25) (layer F.Cu) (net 33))
 (segment (start 134.62 133.35) (end 132.529999 131.259999) (width 0.25) (layer F.Cu) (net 33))
 (segment (start 132.605 118.5) (end 134.105 118.5) (width 0.25) (layer F.Cu) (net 33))
 (segment (start 131.259999 119.845001) (end 132.605 118.5) (width 0.25) (layer F.Cu) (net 33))
 (segment (start 131.259999 131.259999) (end 131.259999 119.845001) (width 0.25) (layer F.Cu) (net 33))
 (segment (start 142.845 138.43) (end 140.305 140.97) (width 0.25) (layer F.Cu) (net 35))
 (segment (start 153.67 138.43) (end 142.845 138.43) (width 0.25) (layer F.Cu) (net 35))
 (segment (start 142.845 138.43) (end 142.503608 138.43) (width 0.25) (layer F.Cu) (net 35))
 (segment (start 137.610009 133.536401) (end 137.610009 133.35) (width 0.25) (layer F.Cu) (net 35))
 (segment (start 142.503608 138.43) (end 137.610009 133.536401) (width 0.25) (layer F.Cu) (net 35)))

